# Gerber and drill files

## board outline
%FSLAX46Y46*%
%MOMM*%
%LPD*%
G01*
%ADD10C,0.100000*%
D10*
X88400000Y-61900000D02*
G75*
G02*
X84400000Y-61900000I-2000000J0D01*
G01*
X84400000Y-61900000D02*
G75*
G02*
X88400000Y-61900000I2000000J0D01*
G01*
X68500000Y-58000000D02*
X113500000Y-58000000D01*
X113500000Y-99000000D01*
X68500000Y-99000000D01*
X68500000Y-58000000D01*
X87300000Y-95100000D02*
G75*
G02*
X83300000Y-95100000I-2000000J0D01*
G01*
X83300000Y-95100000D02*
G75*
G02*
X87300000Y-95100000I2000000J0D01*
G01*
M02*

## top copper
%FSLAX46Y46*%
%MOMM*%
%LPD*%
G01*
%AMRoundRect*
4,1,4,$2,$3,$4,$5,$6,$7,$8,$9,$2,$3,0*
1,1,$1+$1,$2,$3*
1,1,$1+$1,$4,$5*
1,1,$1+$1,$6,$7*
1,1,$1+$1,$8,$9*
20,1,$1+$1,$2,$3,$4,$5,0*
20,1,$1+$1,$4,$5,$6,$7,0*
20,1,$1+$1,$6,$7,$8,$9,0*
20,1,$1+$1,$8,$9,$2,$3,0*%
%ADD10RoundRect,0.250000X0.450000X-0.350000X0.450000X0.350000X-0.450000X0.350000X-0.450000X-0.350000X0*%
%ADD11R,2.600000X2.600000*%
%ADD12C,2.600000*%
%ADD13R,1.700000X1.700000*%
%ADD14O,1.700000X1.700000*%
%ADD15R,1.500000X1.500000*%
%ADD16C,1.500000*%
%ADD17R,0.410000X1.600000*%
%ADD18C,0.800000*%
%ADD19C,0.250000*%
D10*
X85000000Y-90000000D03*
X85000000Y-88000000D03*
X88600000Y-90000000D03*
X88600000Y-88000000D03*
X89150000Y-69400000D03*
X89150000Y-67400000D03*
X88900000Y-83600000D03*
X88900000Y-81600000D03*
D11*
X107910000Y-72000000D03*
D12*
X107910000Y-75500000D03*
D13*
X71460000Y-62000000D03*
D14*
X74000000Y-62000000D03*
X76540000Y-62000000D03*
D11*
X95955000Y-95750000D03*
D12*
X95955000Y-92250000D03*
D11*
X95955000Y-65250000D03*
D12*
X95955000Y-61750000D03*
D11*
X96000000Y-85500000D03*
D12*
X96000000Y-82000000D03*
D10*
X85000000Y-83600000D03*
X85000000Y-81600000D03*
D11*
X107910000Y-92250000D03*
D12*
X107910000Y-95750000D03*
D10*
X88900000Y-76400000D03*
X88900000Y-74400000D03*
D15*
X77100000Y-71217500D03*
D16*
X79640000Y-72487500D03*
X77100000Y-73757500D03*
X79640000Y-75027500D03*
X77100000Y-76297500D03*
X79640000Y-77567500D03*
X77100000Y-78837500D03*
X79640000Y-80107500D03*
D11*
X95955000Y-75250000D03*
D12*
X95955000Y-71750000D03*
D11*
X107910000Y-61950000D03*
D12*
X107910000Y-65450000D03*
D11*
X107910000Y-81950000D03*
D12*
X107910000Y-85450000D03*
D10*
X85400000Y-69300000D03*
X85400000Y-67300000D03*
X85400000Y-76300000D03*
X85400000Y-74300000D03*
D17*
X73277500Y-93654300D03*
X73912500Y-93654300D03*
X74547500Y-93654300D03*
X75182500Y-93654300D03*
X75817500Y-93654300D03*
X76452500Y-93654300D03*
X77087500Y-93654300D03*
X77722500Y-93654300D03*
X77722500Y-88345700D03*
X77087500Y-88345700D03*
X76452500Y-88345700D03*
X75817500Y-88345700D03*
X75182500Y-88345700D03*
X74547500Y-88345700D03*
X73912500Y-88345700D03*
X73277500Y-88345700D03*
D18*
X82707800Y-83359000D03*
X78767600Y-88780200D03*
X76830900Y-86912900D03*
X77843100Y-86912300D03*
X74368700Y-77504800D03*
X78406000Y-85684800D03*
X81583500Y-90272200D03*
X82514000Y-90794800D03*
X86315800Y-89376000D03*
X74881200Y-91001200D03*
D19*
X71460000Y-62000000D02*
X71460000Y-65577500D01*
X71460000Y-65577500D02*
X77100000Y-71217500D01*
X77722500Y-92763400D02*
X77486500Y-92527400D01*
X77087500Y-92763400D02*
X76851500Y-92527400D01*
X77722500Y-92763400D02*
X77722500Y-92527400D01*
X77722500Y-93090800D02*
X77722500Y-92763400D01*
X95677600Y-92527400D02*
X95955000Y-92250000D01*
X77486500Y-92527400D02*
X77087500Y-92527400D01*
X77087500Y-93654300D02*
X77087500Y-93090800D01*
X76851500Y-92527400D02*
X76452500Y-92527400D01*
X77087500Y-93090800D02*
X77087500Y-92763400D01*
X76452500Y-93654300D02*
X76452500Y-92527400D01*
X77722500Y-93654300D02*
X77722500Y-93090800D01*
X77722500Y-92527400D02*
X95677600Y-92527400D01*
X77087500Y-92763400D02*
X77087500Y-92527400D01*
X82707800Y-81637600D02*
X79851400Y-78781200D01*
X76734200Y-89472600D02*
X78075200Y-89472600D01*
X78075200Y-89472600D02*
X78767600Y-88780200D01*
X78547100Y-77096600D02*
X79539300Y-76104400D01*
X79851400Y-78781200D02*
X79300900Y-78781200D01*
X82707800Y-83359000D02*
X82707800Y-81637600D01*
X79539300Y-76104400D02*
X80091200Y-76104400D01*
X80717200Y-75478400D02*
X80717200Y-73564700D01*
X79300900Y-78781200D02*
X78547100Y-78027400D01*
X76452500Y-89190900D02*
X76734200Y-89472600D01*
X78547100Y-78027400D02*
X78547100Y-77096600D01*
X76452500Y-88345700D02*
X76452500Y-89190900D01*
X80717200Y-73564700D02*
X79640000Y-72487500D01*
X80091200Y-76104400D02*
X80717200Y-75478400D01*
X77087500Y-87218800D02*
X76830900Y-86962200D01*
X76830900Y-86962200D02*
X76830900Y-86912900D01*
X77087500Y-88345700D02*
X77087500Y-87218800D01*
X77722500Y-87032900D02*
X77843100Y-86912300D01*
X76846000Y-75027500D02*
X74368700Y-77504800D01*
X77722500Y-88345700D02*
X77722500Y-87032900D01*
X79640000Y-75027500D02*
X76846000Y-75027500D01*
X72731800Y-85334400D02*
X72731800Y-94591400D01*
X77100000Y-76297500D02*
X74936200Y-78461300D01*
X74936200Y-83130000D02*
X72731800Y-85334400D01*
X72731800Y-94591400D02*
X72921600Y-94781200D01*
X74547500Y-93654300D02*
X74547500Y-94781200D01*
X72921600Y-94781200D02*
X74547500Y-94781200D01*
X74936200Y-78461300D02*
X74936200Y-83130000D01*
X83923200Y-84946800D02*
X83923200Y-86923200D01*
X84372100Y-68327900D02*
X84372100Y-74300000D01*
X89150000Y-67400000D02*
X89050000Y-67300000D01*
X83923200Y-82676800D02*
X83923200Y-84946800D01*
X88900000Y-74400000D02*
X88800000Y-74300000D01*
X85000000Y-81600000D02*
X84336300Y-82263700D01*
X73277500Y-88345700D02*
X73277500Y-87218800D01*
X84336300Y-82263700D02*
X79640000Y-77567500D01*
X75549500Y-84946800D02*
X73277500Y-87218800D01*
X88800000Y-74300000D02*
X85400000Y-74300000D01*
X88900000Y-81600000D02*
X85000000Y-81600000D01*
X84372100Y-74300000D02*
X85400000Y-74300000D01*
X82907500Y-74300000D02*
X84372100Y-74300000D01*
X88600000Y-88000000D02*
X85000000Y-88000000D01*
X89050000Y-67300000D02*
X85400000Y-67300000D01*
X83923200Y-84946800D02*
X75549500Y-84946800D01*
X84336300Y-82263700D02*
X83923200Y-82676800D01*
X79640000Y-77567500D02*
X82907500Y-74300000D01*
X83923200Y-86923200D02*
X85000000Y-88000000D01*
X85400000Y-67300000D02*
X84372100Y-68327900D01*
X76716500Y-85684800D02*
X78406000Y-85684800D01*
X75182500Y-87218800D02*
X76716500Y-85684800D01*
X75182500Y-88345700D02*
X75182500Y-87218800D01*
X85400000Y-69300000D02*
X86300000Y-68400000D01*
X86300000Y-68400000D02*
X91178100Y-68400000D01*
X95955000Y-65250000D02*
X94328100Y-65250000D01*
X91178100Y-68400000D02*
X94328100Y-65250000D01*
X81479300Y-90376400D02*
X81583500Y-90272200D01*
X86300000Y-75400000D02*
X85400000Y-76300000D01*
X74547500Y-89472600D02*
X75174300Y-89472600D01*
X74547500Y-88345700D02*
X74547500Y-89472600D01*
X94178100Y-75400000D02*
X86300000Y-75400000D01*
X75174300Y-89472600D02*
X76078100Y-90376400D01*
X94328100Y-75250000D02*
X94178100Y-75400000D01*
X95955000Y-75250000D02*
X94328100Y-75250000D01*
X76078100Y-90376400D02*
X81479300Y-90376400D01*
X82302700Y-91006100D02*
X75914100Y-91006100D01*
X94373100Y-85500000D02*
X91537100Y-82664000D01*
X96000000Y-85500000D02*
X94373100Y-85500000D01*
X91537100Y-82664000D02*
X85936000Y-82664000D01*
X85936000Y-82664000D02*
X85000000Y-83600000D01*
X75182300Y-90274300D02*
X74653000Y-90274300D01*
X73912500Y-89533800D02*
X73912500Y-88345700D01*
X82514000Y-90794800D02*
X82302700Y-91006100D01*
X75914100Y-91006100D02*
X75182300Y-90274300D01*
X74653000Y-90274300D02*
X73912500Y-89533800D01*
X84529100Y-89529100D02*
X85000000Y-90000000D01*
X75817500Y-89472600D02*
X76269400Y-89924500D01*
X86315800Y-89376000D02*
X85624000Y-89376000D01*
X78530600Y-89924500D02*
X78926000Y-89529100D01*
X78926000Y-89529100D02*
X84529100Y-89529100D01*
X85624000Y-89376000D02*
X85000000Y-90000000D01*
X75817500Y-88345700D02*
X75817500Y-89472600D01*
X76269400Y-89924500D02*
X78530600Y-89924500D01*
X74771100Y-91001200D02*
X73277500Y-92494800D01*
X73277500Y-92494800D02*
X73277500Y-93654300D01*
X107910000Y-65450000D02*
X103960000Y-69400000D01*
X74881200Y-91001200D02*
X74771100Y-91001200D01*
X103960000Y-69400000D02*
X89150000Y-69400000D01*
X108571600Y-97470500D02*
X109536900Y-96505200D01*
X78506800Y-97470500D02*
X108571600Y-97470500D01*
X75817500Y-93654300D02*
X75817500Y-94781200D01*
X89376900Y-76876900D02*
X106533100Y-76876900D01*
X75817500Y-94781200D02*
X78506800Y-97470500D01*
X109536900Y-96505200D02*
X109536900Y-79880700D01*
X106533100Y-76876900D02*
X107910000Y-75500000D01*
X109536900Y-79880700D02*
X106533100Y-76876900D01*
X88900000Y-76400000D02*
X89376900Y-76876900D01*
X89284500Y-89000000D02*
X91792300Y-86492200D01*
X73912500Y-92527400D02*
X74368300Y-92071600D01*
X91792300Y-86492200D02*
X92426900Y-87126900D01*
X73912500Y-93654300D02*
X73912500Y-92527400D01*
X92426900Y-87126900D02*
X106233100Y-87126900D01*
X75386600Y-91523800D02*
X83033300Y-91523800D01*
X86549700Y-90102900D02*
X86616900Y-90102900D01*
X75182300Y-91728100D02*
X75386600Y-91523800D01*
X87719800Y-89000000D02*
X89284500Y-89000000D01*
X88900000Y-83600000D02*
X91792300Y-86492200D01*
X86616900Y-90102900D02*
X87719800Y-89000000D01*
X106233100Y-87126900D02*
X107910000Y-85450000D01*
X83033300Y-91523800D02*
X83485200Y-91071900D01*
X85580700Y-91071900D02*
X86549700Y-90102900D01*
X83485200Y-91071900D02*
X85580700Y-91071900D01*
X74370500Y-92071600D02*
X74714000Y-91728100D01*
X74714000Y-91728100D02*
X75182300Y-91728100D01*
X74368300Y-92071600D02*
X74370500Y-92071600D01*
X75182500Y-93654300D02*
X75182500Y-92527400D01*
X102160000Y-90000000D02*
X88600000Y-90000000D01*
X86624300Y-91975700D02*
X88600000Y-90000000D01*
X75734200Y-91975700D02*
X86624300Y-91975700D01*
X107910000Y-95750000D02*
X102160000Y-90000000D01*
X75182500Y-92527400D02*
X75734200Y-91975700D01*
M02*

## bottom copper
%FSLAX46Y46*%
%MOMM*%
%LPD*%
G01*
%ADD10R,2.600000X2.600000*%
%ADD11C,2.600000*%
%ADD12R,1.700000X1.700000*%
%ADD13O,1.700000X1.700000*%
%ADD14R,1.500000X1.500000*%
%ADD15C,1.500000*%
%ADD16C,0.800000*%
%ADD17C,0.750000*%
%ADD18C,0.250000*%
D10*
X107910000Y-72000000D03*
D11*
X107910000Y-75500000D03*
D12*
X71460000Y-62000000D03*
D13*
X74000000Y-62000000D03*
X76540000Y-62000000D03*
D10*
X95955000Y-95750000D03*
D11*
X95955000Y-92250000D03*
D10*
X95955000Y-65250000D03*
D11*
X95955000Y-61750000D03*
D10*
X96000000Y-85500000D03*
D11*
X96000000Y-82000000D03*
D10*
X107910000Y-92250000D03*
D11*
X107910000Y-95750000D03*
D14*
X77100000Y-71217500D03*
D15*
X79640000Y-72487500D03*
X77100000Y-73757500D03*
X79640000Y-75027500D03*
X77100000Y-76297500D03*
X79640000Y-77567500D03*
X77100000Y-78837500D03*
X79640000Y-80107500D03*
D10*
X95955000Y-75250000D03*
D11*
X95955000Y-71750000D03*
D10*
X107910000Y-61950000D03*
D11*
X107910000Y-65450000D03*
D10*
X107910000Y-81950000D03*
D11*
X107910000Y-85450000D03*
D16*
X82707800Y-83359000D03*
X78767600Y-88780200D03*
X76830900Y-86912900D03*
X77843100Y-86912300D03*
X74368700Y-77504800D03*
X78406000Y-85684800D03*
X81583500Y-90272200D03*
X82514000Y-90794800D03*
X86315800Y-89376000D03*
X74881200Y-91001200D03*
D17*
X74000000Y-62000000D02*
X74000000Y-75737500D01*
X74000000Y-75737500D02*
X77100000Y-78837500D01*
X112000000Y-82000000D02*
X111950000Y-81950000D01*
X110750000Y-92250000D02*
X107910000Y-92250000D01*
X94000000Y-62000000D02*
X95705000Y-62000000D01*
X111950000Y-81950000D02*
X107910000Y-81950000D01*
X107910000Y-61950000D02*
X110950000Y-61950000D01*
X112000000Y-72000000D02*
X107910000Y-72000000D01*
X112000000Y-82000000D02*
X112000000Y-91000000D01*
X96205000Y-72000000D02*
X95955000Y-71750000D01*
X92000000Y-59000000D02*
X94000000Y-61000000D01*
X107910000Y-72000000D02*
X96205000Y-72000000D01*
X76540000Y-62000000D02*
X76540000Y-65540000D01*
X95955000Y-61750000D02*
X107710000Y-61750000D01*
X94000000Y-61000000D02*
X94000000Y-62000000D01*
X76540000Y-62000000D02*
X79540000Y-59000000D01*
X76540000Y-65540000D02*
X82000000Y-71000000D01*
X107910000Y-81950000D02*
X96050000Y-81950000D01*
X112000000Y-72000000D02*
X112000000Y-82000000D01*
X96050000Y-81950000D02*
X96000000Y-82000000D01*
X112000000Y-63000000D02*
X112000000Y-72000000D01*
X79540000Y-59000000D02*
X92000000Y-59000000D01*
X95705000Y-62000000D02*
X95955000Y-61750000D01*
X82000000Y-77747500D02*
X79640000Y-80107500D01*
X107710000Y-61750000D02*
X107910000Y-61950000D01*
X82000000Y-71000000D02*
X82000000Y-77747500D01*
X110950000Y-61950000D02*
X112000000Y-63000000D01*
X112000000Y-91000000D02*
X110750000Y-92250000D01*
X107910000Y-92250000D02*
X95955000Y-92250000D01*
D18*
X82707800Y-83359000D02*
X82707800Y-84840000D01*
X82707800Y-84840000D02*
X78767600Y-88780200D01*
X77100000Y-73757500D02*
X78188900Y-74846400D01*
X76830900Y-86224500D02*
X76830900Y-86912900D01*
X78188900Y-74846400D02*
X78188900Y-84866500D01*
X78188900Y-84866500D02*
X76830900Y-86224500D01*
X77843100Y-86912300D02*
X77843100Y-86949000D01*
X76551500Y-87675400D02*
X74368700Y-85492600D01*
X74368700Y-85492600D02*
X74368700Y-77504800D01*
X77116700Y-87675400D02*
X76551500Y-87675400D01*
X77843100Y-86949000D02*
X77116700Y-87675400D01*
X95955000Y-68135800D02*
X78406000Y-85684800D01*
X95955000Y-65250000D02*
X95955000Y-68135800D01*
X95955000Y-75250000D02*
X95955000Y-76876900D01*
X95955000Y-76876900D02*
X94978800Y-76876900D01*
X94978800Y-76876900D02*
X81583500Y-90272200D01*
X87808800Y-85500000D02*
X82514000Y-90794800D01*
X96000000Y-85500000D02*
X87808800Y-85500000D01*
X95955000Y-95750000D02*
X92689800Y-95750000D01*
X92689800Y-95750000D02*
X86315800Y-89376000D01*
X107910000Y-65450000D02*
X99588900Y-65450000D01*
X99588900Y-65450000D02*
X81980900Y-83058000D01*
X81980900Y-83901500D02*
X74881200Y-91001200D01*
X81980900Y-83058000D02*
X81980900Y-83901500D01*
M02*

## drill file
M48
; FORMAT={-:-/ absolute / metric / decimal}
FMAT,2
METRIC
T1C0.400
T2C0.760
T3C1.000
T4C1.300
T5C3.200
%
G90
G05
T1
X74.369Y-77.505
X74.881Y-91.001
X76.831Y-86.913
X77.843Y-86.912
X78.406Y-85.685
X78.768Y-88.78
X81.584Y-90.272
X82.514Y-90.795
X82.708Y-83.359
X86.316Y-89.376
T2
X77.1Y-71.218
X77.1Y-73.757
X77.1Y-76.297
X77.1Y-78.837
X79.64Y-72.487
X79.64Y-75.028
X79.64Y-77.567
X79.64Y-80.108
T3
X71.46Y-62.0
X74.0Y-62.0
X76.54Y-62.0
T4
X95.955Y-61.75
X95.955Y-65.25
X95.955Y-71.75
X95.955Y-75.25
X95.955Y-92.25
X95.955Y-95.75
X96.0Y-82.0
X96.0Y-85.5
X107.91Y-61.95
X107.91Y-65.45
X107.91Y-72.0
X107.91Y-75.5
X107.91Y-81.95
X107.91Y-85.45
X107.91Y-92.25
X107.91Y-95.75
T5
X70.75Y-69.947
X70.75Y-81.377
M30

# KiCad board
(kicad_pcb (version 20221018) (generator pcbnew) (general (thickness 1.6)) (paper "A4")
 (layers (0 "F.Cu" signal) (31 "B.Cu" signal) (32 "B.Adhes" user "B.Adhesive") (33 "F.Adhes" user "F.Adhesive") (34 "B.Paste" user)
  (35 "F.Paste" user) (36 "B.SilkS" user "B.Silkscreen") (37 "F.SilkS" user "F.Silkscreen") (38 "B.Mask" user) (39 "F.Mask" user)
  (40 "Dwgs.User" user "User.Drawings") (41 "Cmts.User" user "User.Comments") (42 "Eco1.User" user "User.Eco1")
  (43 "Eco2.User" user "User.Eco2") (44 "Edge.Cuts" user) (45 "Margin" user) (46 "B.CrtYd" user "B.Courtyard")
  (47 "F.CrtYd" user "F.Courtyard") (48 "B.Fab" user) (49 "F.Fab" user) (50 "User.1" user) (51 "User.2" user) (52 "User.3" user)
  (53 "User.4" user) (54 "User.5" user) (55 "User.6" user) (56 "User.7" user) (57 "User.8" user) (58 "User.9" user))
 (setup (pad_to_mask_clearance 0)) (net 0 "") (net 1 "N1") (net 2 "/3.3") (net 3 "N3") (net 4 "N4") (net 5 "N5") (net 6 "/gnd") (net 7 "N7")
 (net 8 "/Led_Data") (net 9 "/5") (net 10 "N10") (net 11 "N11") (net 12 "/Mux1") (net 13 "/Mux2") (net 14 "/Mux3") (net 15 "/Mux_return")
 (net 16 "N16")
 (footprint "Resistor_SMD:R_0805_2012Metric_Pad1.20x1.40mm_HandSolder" (layer "F.Cu") (at 85 89 90)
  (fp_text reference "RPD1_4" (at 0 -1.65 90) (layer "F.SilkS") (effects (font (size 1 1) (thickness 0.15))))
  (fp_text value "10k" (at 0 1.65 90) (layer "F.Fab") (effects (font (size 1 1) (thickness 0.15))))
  (pad "1" smd roundrect (at -1 0 90) (size 1.2 1.4) (layers "F.Cu" "F.Paste" "F.Mask") (roundrect_rratio 0.2083333333) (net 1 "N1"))
  (pad "2" smd roundrect (at 1 0 90) (size 1.2 1.4) (layers "F.Cu" "F.Paste" "F.Mask") (roundrect_rratio 0.2083333333) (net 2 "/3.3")))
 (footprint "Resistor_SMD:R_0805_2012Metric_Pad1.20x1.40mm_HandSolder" (layer "F.Cu") (at 88.6 89 90)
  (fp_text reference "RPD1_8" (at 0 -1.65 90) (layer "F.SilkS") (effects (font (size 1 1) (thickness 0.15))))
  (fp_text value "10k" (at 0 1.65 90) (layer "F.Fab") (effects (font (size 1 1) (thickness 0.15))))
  (pad "1" smd roundrect (at -1 0 90) (size 1.2 1.4) (layers "F.Cu" "F.Paste" "F.Mask") (roundrect_rratio 0.2083333333) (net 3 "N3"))
  (pad "2" smd roundrect (at 1 0 90) (size 1.2 1.4) (layers "F.Cu" "F.Paste" "F.Mask") (roundrect_rratio 0.2083333333) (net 2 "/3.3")))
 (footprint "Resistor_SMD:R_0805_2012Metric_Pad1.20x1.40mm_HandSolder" (layer "F.Cu") (at 89.15 68.4 90)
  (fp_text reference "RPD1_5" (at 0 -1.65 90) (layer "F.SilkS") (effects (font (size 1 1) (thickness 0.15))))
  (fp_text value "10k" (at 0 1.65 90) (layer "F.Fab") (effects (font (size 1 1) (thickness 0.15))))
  (pad "1" smd roundrect (at -1 0 90) (size 1.2 1.4) (layers "F.Cu" "F.Paste" "F.Mask") (roundrect_rratio 0.2083333333) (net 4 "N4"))
  (pad "2" smd roundrect (at 1 0 90) (size 1.2 1.4) (layers "F.Cu" "F.Paste" "F.Mask") (roundrect_rratio 0.2083333333) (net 2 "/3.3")))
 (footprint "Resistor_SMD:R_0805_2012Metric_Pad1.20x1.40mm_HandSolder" (layer "F.Cu") (at 88.9 82.6 90)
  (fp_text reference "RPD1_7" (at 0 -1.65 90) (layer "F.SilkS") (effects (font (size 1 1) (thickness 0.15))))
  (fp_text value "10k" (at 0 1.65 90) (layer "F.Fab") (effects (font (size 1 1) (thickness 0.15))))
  (pad "1" smd roundrect (at -1 0 90) (size 1.2 1.4) (layers "F.Cu" "F.Paste" "F.Mask") (roundrect_rratio 0.2083333333) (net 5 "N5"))
  (pad "2" smd roundrect (at 1 0 90) (size 1.2 1.4) (layers "F.Cu" "F.Paste" "F.Mask") (roundrect_rratio 0.2083333333) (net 2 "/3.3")))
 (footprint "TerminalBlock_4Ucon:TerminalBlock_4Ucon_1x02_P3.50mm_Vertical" (layer "F.Cu") (at 107.91 72 -90)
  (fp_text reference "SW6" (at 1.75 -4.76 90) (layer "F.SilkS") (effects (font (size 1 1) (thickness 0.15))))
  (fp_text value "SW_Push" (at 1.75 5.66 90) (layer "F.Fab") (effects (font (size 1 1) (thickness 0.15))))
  (pad "1" thru_hole rect (at 0 0 270) (size 2.6 2.6) (drill 1.3) (layers "*.Cu" "*.Mask") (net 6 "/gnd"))
  (pad "2" thru_hole circle (at 3.5 0 270) (size 2.6 2.6) (drill 1.3) (layers "*.Cu" "*.Mask") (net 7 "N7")))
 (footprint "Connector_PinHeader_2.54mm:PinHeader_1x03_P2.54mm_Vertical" (layer "F.Cu") (at 71.46 62 90)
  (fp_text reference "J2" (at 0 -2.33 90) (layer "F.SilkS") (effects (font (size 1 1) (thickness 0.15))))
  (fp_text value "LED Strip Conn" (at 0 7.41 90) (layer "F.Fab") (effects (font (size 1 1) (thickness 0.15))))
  (pad "1" thru_hole rect (at 0 0 90) (size 1.7 1.7) (drill 1) (layers "*.Cu" "*.Mask") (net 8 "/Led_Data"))
  (pad "2" thru_hole oval (at 0 2.54 90) (size 1.7 1.7) (drill 1) (layers "*.Cu" "*.Mask") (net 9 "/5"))
  (pad "3" thru_hole oval (at 0 5.08 90) (size 1.7 1.7) (drill 1) (layers "*.Cu" "*.Mask") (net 6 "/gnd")))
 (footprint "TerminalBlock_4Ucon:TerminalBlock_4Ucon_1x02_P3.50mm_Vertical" (layer "F.Cu") (at 95.955 95.75 90)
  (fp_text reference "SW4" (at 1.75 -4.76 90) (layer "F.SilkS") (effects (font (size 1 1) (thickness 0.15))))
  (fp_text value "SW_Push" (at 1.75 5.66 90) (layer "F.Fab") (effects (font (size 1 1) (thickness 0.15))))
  (pad "1" thru_hole rect (at 0 0 90) (size 2.6 2.6) (drill 1.3) (layers "*.Cu" "*.Mask") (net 1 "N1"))
  (pad "2" thru_hole circle (at 3.5 0 90) (size 2.6 2.6) (drill 1.3) (layers "*.Cu" "*.Mask") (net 6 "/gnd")))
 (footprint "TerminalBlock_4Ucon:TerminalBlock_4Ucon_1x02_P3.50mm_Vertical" (layer "F.Cu") (at 95.955 65.25 90)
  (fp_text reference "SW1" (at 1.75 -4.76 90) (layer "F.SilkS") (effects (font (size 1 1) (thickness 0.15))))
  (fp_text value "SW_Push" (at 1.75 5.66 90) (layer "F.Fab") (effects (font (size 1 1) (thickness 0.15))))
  (pad "1" thru_hole rect (at 0 0 90) (size 2.6 2.6) (drill 1.3) (layers "*.Cu" "*.Mask") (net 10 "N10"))
  (pad "2" thru_hole circle (at 3.5 0 90) (size 2.6 2.6) (drill 1.3) (layers "*.Cu" "*.Mask") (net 6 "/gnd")))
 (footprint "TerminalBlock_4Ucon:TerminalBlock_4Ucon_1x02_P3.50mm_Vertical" (layer "F.Cu") (at 96 85.5 90)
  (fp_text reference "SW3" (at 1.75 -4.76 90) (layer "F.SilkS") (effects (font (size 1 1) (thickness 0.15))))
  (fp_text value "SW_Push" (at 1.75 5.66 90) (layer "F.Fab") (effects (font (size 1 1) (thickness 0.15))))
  (pad "1" thru_hole rect (at 0 0 90) (size 2.6 2.6) (drill 1.3) (layers "*.Cu" "*.Mask") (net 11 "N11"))
  (pad "2" thru_hole circle (at 3.5 0 90) (size 2.6 2.6) (drill 1.3) (layers "*.Cu" "*.Mask") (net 6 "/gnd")))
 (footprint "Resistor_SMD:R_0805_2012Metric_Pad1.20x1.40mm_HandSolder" (layer "F.Cu") (at 85 82.6 90)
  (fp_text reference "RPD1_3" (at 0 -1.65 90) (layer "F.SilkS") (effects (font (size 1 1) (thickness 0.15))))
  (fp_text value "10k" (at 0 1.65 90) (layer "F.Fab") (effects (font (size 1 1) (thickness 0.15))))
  (pad "1" smd roundrect (at -1 0 90) (size 1.2 1.4) (layers "F.Cu" "F.Paste" "F.Mask") (roundrect_rratio 0.2083333333) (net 11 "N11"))
  (pad "2" smd roundrect (at 1 0 90) (size 1.2 1.4) (layers "F.Cu" "F.Paste" "F.Mask") (roundrect_rratio 0.2083333333) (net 2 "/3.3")))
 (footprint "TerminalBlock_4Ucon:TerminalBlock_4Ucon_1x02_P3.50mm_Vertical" (layer "F.Cu") (at 107.91 92.25 -90)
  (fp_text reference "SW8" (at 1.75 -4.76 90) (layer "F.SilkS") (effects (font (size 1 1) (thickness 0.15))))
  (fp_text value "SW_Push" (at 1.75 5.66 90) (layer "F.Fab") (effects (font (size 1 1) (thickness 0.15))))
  (pad "1" thru_hole rect (at 0 0 270) (size 2.6 2.6) (drill 1.3) (layers "*.Cu" "*.Mask") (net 6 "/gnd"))
  (pad "2" thru_hole circle (at 3.5 0 270) (size 2.6 2.6) (drill 1.3) (layers "*.Cu" "*.Mask") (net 3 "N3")))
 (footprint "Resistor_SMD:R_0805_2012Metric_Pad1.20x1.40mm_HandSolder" (layer "F.Cu") (at 88.9 75.4 90)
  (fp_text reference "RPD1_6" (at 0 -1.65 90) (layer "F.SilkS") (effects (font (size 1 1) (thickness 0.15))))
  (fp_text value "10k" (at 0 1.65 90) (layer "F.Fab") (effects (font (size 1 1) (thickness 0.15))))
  (pad "1" smd roundrect (at -1 0 90) (size 1.2 1.4) (layers "F.Cu" "F.Paste" "F.Mask") (roundrect_rratio 0.2083333333) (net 7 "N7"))
  (pad "2" smd roundrect (at 1 0 90) (size 1.2 1.4) (layers "F.Cu" "F.Paste" "F.Mask") (roundrect_rratio 0.2083333333) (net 2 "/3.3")))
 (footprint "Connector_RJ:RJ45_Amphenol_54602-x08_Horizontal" (layer "F.Cu") (at 77.1 71.2175 -90)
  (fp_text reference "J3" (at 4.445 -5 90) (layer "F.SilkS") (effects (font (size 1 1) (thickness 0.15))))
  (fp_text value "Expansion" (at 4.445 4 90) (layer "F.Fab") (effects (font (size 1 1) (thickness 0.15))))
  (pad "" np_thru_hole circle (at -1.27 6.35 270) (size 3.2 3.2) (drill 3.2) (layers "*.Cu" "*.Mask"))
  (pad "" np_thru_hole circle (at 10.16 6.35 270) (size 3.2 3.2) (drill 3.2) (layers "*.Cu" "*.Mask"))
  (pad "1" thru_hole rect (at 0 0 270) (size 1.5 1.5) (drill 0.76) (layers "*.Cu" "*.Mask") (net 8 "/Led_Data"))
  (pad "2" thru_hole circle (at 1.27 -2.54 270) (size 1.5 1.5) (drill 0.76) (layers "*.Cu" "*.Mask") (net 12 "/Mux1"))
  (pad "3" thru_hole circle (at 2.54 0 270) (size 1.5 1.5) (drill 0.76) (layers "*.Cu" "*.Mask") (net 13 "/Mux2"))
  (pad "4" thru_hole circle (at 3.81 -2.54 270) (size 1.5 1.5) (drill 0.76) (layers "*.Cu" "*.Mask") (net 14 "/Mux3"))
  (pad "5" thru_hole circle (at 5.08 0 270) (size 1.5 1.5) (drill 0.76) (layers "*.Cu" "*.Mask") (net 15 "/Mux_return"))
  (pad "6" thru_hole circle (at 6.35 -2.54 270) (size 1.5 1.5) (drill 0.76) (layers "*.Cu" "*.Mask") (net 2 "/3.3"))
  (pad "7" thru_hole circle (at 7.62 0 270) (size 1.5 1.5) (drill 0.76) (layers "*.Cu" "*.Mask") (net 9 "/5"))
  (pad "8" thru_hole circle (at 8.89 -2.54 270) (size 1.5 1.5) (drill 0.76) (layers "*.Cu" "*.Mask") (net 6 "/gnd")))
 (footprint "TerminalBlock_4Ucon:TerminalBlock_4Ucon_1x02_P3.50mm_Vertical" (layer "F.Cu") (at 95.955 75.25 90)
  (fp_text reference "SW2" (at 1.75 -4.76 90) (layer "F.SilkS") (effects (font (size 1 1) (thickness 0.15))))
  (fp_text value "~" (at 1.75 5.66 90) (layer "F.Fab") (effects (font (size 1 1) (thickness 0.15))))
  (pad "1" thru_hole rect (at 0 0 90) (size 2.6 2.6) (drill 1.3) (layers "*.Cu" "*.Mask") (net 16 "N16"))
  (pad "2" thru_hole circle (at 3.5 0 90) (size 2.6 2.6) (drill 1.3) (layers "*.Cu" "*.Mask") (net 6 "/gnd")))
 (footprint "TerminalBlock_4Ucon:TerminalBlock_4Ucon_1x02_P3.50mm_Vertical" (layer "F.Cu") (at 107.91 61.95 -90)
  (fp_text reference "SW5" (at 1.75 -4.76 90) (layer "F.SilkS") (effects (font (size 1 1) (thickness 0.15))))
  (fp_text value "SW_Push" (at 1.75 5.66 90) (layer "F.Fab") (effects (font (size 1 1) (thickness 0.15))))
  (pad "1" thru_hole rect (at 0 0 270) (size 2.6 2.6) (drill 1.3) (layers "*.Cu" "*.Mask") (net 6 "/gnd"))
  (pad "2" thru_hole circle (at 3.5 0 270) (size 2.6 2.6) (drill 1.3) (layers "*.Cu" "*.Mask") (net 4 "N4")))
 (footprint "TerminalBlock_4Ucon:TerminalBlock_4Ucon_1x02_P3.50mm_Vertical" (layer "F.Cu") (at 107.91 81.95 -90)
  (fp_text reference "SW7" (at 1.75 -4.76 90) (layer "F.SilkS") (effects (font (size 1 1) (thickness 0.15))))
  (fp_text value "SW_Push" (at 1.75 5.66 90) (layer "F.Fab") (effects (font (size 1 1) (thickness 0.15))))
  (pad "1" thru_hole rect (at 0 0 270) (size 2.6 2.6) (drill 1.3) (layers "*.Cu" "*.Mask") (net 6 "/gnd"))
  (pad "2" thru_hole circle (at 3.5 0 270) (size 2.6 2.6) (drill 1.3) (layers "*.Cu" "*.Mask") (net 5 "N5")))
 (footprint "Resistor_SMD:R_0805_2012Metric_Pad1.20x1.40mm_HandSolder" (layer "F.Cu") (at 85.4 68.3 90)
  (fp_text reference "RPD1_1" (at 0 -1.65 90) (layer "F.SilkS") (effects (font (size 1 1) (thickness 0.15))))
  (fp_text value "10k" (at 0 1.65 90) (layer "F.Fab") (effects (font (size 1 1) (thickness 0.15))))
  (pad "1" smd roundrect (at -1 0 90) (size 1.2 1.4) (layers "F.Cu" "F.Paste" "F.Mask") (roundrect_rratio 0.2083333333) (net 10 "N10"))
  (pad "2" smd roundrect (at 1 0 90) (size 1.2 1.4) (layers "F.Cu" "F.Paste" "F.Mask") (roundrect_rratio 0.2083333333) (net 2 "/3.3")))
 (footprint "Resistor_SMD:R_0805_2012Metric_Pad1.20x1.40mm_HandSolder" (layer "F.Cu") (at 85.4 75.3 90)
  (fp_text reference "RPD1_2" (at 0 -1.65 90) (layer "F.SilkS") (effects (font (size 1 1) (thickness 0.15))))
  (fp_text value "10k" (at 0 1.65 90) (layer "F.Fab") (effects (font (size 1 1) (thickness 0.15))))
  (pad "1" smd roundrect (at -1 0 90) (size 1.2 1.4) (layers "F.Cu" "F.Paste" "F.Mask") (roundrect_rratio 0.2083333333) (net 16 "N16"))
  (pad "2" smd roundrect (at 1 0 90) (size 1.2 1.4) (layers "F.Cu" "F.Paste" "F.Mask") (roundrect_rratio 0.2083333333) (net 2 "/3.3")))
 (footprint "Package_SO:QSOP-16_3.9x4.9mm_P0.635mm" (layer "F.Cu") (at 75.5 91 90)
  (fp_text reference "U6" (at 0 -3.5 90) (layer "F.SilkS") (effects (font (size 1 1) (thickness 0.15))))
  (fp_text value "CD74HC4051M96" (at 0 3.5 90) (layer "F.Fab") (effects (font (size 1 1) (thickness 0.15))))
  (pad "1" smd rect (at -2.6543 -2.2225 90) (size 1.6 0.41) (layers "F.Cu" "F.Paste" "F.Mask") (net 4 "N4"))
  (pad "2" smd rect (at -2.6543 -1.5875 90) (size 1.6 0.41) (layers "F.Cu" "F.Paste" "F.Mask") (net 5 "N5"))
  (pad "3" smd rect (at -2.6543 -0.9525 90) (size 1.6 0.41) (layers "F.Cu" "F.Paste" "F.Mask") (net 15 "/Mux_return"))
  (pad "4" smd rect (at -2.6543 -0.3175 90) (size 1.6 0.41) (layers "F.Cu" "F.Paste" "F.Mask") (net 3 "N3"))
  (pad "5" smd rect (at -2.6543 0.3175 90) (size 1.6 0.41) (layers "F.Cu" "F.Paste" "F.Mask") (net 7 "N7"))
  (pad "6" smd rect (at -2.6543 0.9525 90) (size 1.6 0.41) (layers "F.Cu" "F.Paste" "F.Mask") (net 6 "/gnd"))
  (pad "7" smd rect (at -2.6543 1.5875 90) (size 1.6 0.41) (layers "F.Cu" "F.Paste" "F.Mask") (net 6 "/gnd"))
  (pad "8" smd rect (at -2.6543 2.2225 90) (size 1.6 0.41) (layers "F.Cu" "F.Paste" "F.Mask") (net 6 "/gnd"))
  (pad "9" smd rect (at 2.6543 2.2225 90) (size 1.6 0.41) (layers "F.Cu" "F.Paste" "F.Mask") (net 14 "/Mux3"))
  (pad "10" smd rect (at 2.6543 1.5875 90) (size 1.6 0.41) (layers "F.Cu" "F.Paste" "F.Mask") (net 13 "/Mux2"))
  (pad "11" smd rect (at 2.6543 0.9525 90) (size 1.6 0.41) (layers "F.Cu" "F.Paste" "F.Mask") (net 12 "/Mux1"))
  (pad "12" smd rect (at 2.6543 0.3175 90) (size 1.6 0.41) (layers "F.Cu" "F.Paste" "F.Mask") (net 1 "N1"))
  (pad "13" smd rect (at 2.6543 -0.3175 90) (size 1.6 0.41) (layers "F.Cu" "F.Paste" "F.Mask") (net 10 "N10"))
  (pad "14" smd rect (at 2.6543 -0.9525 90) (size 1.6 0.41) (layers "F.Cu" "F.Paste" "F.Mask") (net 16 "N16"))
  (pad "15" smd rect (at 2.6543 -1.5875 90) (size 1.6 0.41) (layers "F.Cu" "F.Paste" "F.Mask") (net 11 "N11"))
  (pad "16" smd rect (at 2.6543 -2.2225 90) (size 1.6 0.41) (layers "F.Cu" "F.Paste" "F.Mask") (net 2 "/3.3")))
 (gr_circle (center 86.4 61.9) (end 88.4 61.9) (stroke (width 0.1) (type default)) (fill none) (layer "Edge.Cuts"))
 (gr_rect (start 68.5 58) (end 113.5 99) (stroke (width 0.1) (type default)) (fill none) (layer "Edge.Cuts"))
 (gr_circle (center 85.3 95.1) (end 87.3 95.1) (stroke (width 0.1) (type default)) (fill none) (layer "Edge.Cuts"))
 (segment (start 71.46 62) (end 71.46 65.5775) (width 0.25) (layer "F.Cu") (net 8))
 (segment (start 71.46 65.5775) (end 77.1 71.2175) (width 0.25) (layer "F.Cu") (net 8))
 (segment (start 74 62) (end 74 75.7375) (width 0.75) (layer "B.Cu") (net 9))
 (segment (start 74 75.7375) (end 77.1 78.8375) (width 0.75) (layer "B.Cu") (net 9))
 (segment (start 77.7225 92.7634) (end 77.4865 92.5274) (width 0.25) (layer "F.Cu") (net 6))
 (segment (start 77.0875 92.7634) (end 76.8515 92.5274) (width 0.25) (layer "F.Cu") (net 6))
 (segment (start 77.7225 92.7634) (end 77.7225 92.5274) (width 0.25) (layer "F.Cu") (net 6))
 (segment (start 77.7225 93.0908) (end 77.7225 92.7634) (width 0.25) (layer "F.Cu") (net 6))
 (segment (start 95.6776 92.5274) (end 95.955 92.25) (width 0.25) (layer "F.Cu") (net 6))
 (segment (start 77.4865 92.5274) (end 77.0875 92.5274) (width 0.25) (layer "F.Cu") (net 6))
 (segment (start 77.0875 93.6543) (end 77.0875 93.0908) (width 0.25) (layer "F.Cu") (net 6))
 (segment (start 76.8515 92.5274) (end 76.4525 92.5274) (width 0.25) (layer "F.Cu") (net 6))
 (segment (start 77.0875 93.0908) (end 77.0875 92.7634) (width 0.25) (layer "F.Cu") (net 6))
 (segment (start 76.4525 93.6543) (end 76.4525 92.5274) (width 0.25) (layer "F.Cu") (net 6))
 (segment (start 77.7225 93.6543) (end 77.7225 93.0908) (width 0.25) (layer "F.Cu") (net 6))
 (segment (start 77.7225 92.5274) (end 95.6776 92.5274) (width 0.25) (layer "F.Cu") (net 6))
 (segment (start 77.0875 92.7634) (end 77.0875 92.5274) (width 0.25) (layer "F.Cu") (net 6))
 (segment (start 112 82) (end 111.95 81.95) (width 0.75) (layer "B.Cu") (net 6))
 (segment (start 110.75 92.25) (end 107.91 92.25) (width 0.75) (layer "B.Cu") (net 6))
 (segment (start 94 62) (end 95.705 62) (width 0.75) (layer "B.Cu") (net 6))
 (segment (start 111.95 81.95) (end 107.91 81.95) (width 0.75) (layer "B.Cu") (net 6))
 (segment (start 107.91 61.95) (end 110.95 61.95) (width 0.75) (layer "B.Cu") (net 6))
 (segment (start 112 72) (end 107.91 72) (width 0.75) (layer "B.Cu") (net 6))
 (segment (start 112 82) (end 112 91) (width 0.75) (layer "B.Cu") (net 6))
 (segment (start 96.205 72) (end 95.955 71.75) (width 0.75) (layer "B.Cu") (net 6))
 (segment (start 92 59) (end 94 61) (width 0.75) (layer "B.Cu") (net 6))
 (segment (start 107.91 72) (end 96.205 72) (width 0.75) (layer "B.Cu") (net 6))
 (segment (start 76.54 62) (end 76.54 65.54) (width 0.75) (layer "B.Cu") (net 6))
 (segment (start 95.955 61.75) (end 107.71 61.75) (width 0.75) (layer "B.Cu") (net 6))
 (segment (start 94 61) (end 94 62) (width 0.75) (layer "B.Cu") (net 6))
 (segment (start 76.54 62) (end 79.54 59) (width 0.75) (layer "B.Cu") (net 6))
 (segment (start 76.54 65.54) (end 82 71) (width 0.75) (layer "B.Cu") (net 6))
 (segment (start 107.91 81.95) (end 96.05 81.95) (width 0.75) (layer "B.Cu") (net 6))
 (segment (start 112 72) (end 112 82) (width 0.75) (layer "B.Cu") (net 6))
 (segment (start 96.05 81.95) (end 96 82) (width 0.75) (layer "B.Cu") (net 6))
 (segment (start 112 63) (end 112 72) (width 0.75) (layer "B.Cu") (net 6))
 (segment (start 79.54 59) (end 92 59) (width 0.75) (layer "B.Cu") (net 6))
 (segment (start 95.705 62) (end 95.955 61.75) (width 0.75) (layer "B.Cu") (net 6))
 (segment (start 82 77.7475) (end 79.64 80.1075) (width 0.75) (layer "B.Cu") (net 6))
 (segment (start 107.71 61.75) (end 107.91 61.95) (width 0.75) (layer "B.Cu") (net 6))
 (segment (start 82 71) (end 82 77.7475) (width 0.75) (layer "B.Cu") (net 6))
 (segment (start 110.95 61.95) (end 112 63) (width 0.75) (layer "B.Cu") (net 6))
 (segment (start 112 91) (end 110.75 92.25) (width 0.75) (layer "B.Cu") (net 6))
 (segment (start 107.91 92.25) (end 95.955 92.25) (width 0.75) (layer "B.Cu") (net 6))
 (segment (start 82.7078 81.6376) (end 79.8514 78.7812) (width 0.25) (layer "F.Cu") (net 12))
 (segment (start 76.7342 89.4726) (end 78.0752 89.4726) (width 0.25) (layer "F.Cu") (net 12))
 (segment (start 78.0752 89.4726) (end 78.7676 88.7802) (width 0.25) (layer "F.Cu") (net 12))
 (segment (start 78.5471 77.0966) (end 79.5393 76.1044) (width 0.25) (layer "F.Cu") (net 12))
 (segment (start 79.8514 78.7812) (end 79.3009 78.7812) (width 0.25) (layer "F.Cu") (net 12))
 (segment (start 82.7078 83.359) (end 82.7078 81.6376) (width 0.25) (layer "F.Cu") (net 12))
 (segment (start 79.5393 76.1044) (end 80.0912 76.1044) (width 0.25) (layer "F.Cu") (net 12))
 (segment (start 80.7172 75.4784) (end 80.7172 73.5647) (width 0.25) (layer "F.Cu") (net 12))
 (segment (start 79.3009 78.7812) (end 78.5471 78.0274) (width 0.25) (layer "F.Cu") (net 12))
 (segment (start 76.4525 89.1909) (end 76.7342 89.4726) (width 0.25) (layer "F.Cu") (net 12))
 (segment (start 78.5471 78.0274) (end 78.5471 77.0966) (width 0.25) (layer "F.Cu") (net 12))
 (segment (start 76.4525 88.3457) (end 76.4525 89.1909) (width 0.25) (layer "F.Cu") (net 12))
 (segment (start 80.7172 73.5647) (end 79.64 72.4875) (width 0.25) (layer "F.Cu") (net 12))
 (segment (start 80.0912 76.1044) (end 80.7172 75.4784) (width 0.25) (layer "F.Cu") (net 12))
 (via (at 82.7078 83.359) (size 0.8) (drill 0.4) (layers "F.Cu" "B.Cu") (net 12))
 (via (at 78.7676 88.7802) (size 0.8) (drill 0.4) (layers "F.Cu" "B.Cu") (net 12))
 (segment (start 82.7078 83.359) (end 82.7078 84.84) (width 0.25) (layer "B.Cu") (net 12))
 (segment (start 82.7078 84.84) (end 78.7676 88.7802) (width 0.25) (layer "B.Cu") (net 12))
 (segment (start 77.0875 87.2188) (end 76.8309 86.9622) (width 0.25) (layer "F.Cu") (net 13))
 (segment (start 76.8309 86.9622) (end 76.8309 86.9129) (width 0.25) (layer "F.Cu") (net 13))
 (segment (start 77.0875 88.3457) (end 77.0875 87.2188) (width 0.25) (layer "F.Cu") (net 13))
 (via (at 76.8309 86.9129) (size 0.8) (drill 0.4) (layers "F.Cu" "B.Cu") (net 13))
 (segment (start 77.1 73.7575) (end 78.1889 74.8464) (width 0.25) (layer "B.Cu") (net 13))
 (segment (start 76.8309 86.2245) (end 76.8309 86.9129) (width 0.25) (layer "B.Cu") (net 13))
 (segment (start 78.1889 74.8464) (end 78.1889 84.8665) (width 0.25) (layer "B.Cu") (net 13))
 (segment (start 78.1889 84.8665) (end 76.8309 86.2245) (width 0.25) (layer "B.Cu") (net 13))
 (segment (start 77.7225 87.0329) (end 77.8431 86.9123) (width 0.25) (layer "F.Cu") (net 14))
 (segment (start 76.846 75.0275) (end 74.3687 77.5048) (width 0.25) (layer "F.Cu") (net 14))
 (segment (start 77.7225 88.3457) (end 77.7225 87.0329) (width 0.25) (layer "F.Cu") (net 14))
 (segment (start 79.64 75.0275) (end 76.846 75.0275) (width 0.25) (layer "F.Cu") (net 14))
 (via (at 77.8431 86.9123) (size 0.8) (drill 0.4) (layers "F.Cu" "B.Cu") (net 14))
 (via (at 74.3687 77.5048) (size 0.8) (drill 0.4) (layers "F.Cu" "B.Cu") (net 14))
 (segment (start 77.8431 86.9123) (end 77.8431 86.949) (width 0.25) (layer "B.Cu") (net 14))
 (segment (start 76.5515 87.6754) (end 74.3687 85.4926) (width 0.25) (layer "B.Cu") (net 14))
 (segment (start 74.3687 85.4926) (end 74.3687 77.5048) (width 0.25) (layer "B.Cu") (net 14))
 (segment (start 77.1167 87.6754) (end 76.5515 87.6754) (width 0.25) (layer "B.Cu") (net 14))
 (segment (start 77.8431 86.949) (end 77.1167 87.6754) (width 0.25) (layer "B.Cu") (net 14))
 (segment (start 72.7318 85.3344) (end 72.7318 94.5914) (width 0.25) (layer "F.Cu") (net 15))
 (segment (start 77.1 76.2975) (end 74.9362 78.4613) (width 0.25) (layer "F.Cu") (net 15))
 (segment (start 74.9362 83.13) (end 72.7318 85.3344) (width 0.25) (layer "F.Cu") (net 15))
 (segment (start 72.7318 94.5914) (end 72.9216 94.7812) (width 0.25) (layer "F.Cu") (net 15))
 (segment (start 74.5475 93.6543) (end 74.5475 94.7812) (width 0.25) (layer "F.Cu") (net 15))
 (segment (start 72.9216 94.7812) (end 74.5475 94.7812) (width 0.25) (layer "F.Cu") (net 15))
 (segment (start 74.9362 78.4613) (end 74.9362 83.13) (width 0.25) (layer "F.Cu") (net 15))
 (segment (start 83.9232 84.9468) (end 83.9232 86.9232) (width 0.25) (layer "F.Cu") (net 2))
 (segment (start 84.3721 68.3279) (end 84.3721 74.3) (width 0.25) (layer "F.Cu") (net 2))
 (segment (start 89.15 67.4) (end 89.05 67.3) (width 0.25) (layer "F.Cu") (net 2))
 (segment (start 83.9232 82.6768) (end 83.9232 84.9468) (width 0.25) (layer "F.Cu") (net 2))
 (segment (start 88.9 74.4) (end 88.8 74.3) (width 0.25) (layer "F.Cu") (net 2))
 (segment (start 85 81.6) (end 84.3363 82.2637) (width 0.25) (layer "F.Cu") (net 2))
 (segment (start 73.2775 88.3457) (end 73.2775 87.2188) (width 0.25) (layer "F.Cu") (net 2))
 (segment (start 84.3363 82.2637) (end 79.64 77.5675) (width 0.25) (layer "F.Cu") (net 2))
 (segment (start 75.5495 84.9468) (end 73.2775 87.2188) (width 0.25) (layer "F.Cu") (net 2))
 (segment (start 88.8 74.3) (end 85.4 74.3) (width 0.25) (layer "F.Cu") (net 2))
 (segment (start 88.9 81.6) (end 85 81.6) (width 0.25) (layer "F.Cu") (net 2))
 (segment (start 84.3721 74.3) (end 85.4 74.3) (width 0.25) (layer "F.Cu") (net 2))
 (segment (start 82.9075 74.3) (end 84.3721 74.3) (width 0.25) (layer "F.Cu") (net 2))
 (segment (start 88.6 88) (end 85 88) (width 0.25) (layer "F.Cu") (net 2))
 (segment (start 89.05 67.3) (end 85.4 67.3) (width 0.25) (layer "F.Cu") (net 2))
 (segment (start 83.9232 84.9468) (end 75.5495 84.9468) (width 0.25) (layer "F.Cu") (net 2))
 (segment (start 84.3363 82.2637) (end 83.9232 82.6768) (width 0.25) (layer "F.Cu") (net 2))
 (segment (start 79.64 77.5675) (end 82.9075 74.3) (width 0.25) (layer "F.Cu") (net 2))
 (segment (start 83.9232 86.9232) (end 85 88) (width 0.25) (layer "F.Cu") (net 2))
 (segment (start 85.4 67.3) (end 84.3721 68.3279) (width 0.25) (layer "F.Cu") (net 2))
 (segment (start 76.7165 85.6848) (end 78.406 85.6848) (width 0.25) (layer "F.Cu") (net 10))
 (segment (start 75.1825 87.2188) (end 76.7165 85.6848) (width 0.25) (layer "F.Cu") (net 10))
 (segment (start 75.1825 88.3457) (end 75.1825 87.2188) (width 0.25) (layer "F.Cu") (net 10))
 (segment (start 85.4 69.3) (end 86.3 68.4) (width 0.25) (layer "F.Cu") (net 10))
 (segment (start 86.3 68.4) (end 91.1781 68.4) (width 0.25) (layer "F.Cu") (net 10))
 (segment (start 95.955 65.25) (end 94.3281 65.25) (width 0.25) (layer "F.Cu") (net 10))
 (segment (start 91.1781 68.4) (end 94.3281 65.25) (width 0.25) (layer "F.Cu") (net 10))
 (via (at 78.406 85.6848) (size 0.8) (drill 0.4) (layers "F.Cu" "B.Cu") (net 10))
 (segment (start 95.955 68.1358) (end 78.406 85.6848) (width 0.25) (layer "B.Cu") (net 10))
 (segment (start 95.955 65.25) (end 95.955 68.1358) (width 0.25) (layer "B.Cu") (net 10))
 (segment (start 81.4793 90.3764) (end 81.5835 90.2722) (width 0.25) (layer "F.Cu") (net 16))
 (segment (start 86.3 75.4) (end 85.4 76.3) (width 0.25) (layer "F.Cu") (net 16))
 (segment (start 74.5475 89.4726) (end 75.1743 89.4726) (width 0.25) (layer "F.Cu") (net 16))
 (segment (start 74.5475 88.3457) (end 74.5475 89.4726) (width 0.25) (layer "F.Cu") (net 16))
 (segment (start 94.1781 75.4) (end 86.3 75.4) (width 0.25) (layer "F.Cu") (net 16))
 (segment (start 75.1743 89.4726) (end 76.0781 90.3764) (width 0.25) (layer "F.Cu") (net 16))
 (segment (start 94.3281 75.25) (end 94.1781 75.4) (width 0.25) (layer "F.Cu") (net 16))
 (segment (start 95.955 75.25) (end 94.3281 75.25) (width 0.25) (layer "F.Cu") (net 16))
 (segment (start 76.0781 90.3764) (end 81.4793 90.3764) (width 0.25) (layer "F.Cu") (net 16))
 (via (at 81.5835 90.2722) (size 0.8) (drill 0.4) (layers "F.Cu" "B.Cu") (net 16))
 (segment (start 95.955 75.25) (end 95.955 76.8769) (width 0.25) (layer "B.Cu") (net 16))
 (segment (start 95.955 76.8769) (end 94.9788 76.8769) (width 0.25) (layer "B.Cu") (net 16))
 (segment (start 94.9788 76.8769) (end 81.5835 90.2722) (width 0.25) (layer "B.Cu") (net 16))
 (segment (start 82.3027 91.0061) (end 75.9141 91.0061) (width 0.25) (layer "F.Cu") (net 11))
 (segment (start 94.3731 85.5) (end 91.5371 82.664) (width 0.25) (layer "F.Cu") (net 11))
 (segment (start 96 85.5) (end 94.3731 85.5) (width 0.25) (layer "F.Cu") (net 11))
 (segment (start 91.5371 82.664) (end 85.936 82.664) (width 0.25) (layer "F.Cu") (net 11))
 (segment (start 85.936 82.664) (end 85 83.6) (width 0.25) (layer "F.Cu") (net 11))
 (segment (start 75.1823 90.2743) (end 74.653 90.2743) (width 0.25) (layer "F.Cu") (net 11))
 (segment (start 73.9125 89.5338) (end 73.9125 88.3457) (width 0.25) (layer "F.Cu") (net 11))
 (segment (start 82.514 90.7948) (end 82.3027 91.0061) (width 0.25) (layer "F.Cu") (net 11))
 (segment (start 75.9141 91.0061) (end 75.1823 90.2743) (width 0.25) (layer "F.Cu") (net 11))
 (segment (start 74.653 90.2743) (end 73.9125 89.5338) (width 0.25) (layer "F.Cu") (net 11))
 (via (at 82.514 90.7948) (size 0.8) (drill 0.4) (layers "F.Cu" "B.Cu") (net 11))
 (segment (start 87.8088 85.5) (end 82.514 90.7948) (width 0.25) (layer "B.Cu") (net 11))
 (segment (start 96 85.5) (end 87.8088 85.5) (width 0.25) (layer "B.Cu") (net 11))
 (segment (start 84.5291 89.5291) (end 85 90) (width 0.25) (layer "F.Cu") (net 1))
 (segment (start 75.8175 89.4726) (end 76.2694 89.9245) (width 0.25) (layer "F.Cu") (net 1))
 (segment (start 86.3158 89.376) (end 85.624 89.376) (width 0.25) (layer "F.Cu") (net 1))
 (segment (start 78.5306 89.9245) (end 78.926 89.5291) (width 0.25) (layer "F.Cu") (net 1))
 (segment (start 78.926 89.5291) (end 84.5291 89.5291) (width 0.25) (layer "F.Cu") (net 1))
 (segment (start 85.624 89.376) (end 85 90) (width 0.25) (layer "F.Cu") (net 1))
 (segment (start 75.8175 88.3457) (end 75.8175 89.4726) (width 0.25) (layer "F.Cu") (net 1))
 (segment (start 76.2694 89.9245) (end 78.5306 89.9245) (width 0.25) (layer "F.Cu") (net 1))
 (via (at 86.3158 89.376) (size 0.8) (drill 0.4) (layers "F.Cu" "B.Cu") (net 1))
 (segment (start 95.955 95.75) (end 92.6898 95.75) (width 0.25) (layer "B.Cu") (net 1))
 (segment (start 92.6898 95.75) (end 86.3158 89.376) (width 0.25) (layer "B.Cu") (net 1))
 (segment (start 74.7711 91.0012) (end 73.2775 92.4948) (width 0.25) (layer "F.Cu") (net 4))
 (segment (start 73.2775 92.4948) (end 73.2775 93.6543) (width 0.25) (layer "F.Cu") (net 4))
 (segment (start 107.91 65.45) (end 103.96 69.4) (width 0.25) (layer "F.Cu") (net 4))
 (segment (start 74.8812 91.0012) (end 74.7711 91.0012) (width 0.25) (layer "F.Cu") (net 4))
 (segment (start 103.96 69.4) (end 89.15 69.4) (width 0.25) (layer "F.Cu") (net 4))
 (via (at 74.8812 91.0012) (size 0.8) (drill 0.4) (layers "F.Cu" "B.Cu") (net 4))
 (segment (start 107.91 65.45) (end 99.5889 65.45) (width 0.25) (layer "B.Cu") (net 4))
 (segment (start 99.5889 65.45) (end 81.9809 83.058) (width 0.25) (layer "B.Cu") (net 4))
 (segment (start 81.9809 83.9015) (end 74.8812 91.0012) (width 0.25) (layer "B.Cu") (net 4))
 (segment (start 81.9809 83.058) (end 81.9809 83.9015) (width 0.25) (layer "B.Cu") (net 4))
 (segment (start 108.5716 97.4705) (end 109.5369 96.5052) (width 0.25) (layer "F.Cu") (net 7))
 (segment (start 78.5068 97.4705) (end 108.5716 97.4705) (width 0.25) (layer "F.Cu") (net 7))
 (segment (start 75.8175 93.6543) (end 75.8175 94.7812) (width 0.25) (layer "F.Cu") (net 7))
 (segment (start 89.3769 76.8769) (end 106.5331 76.8769) (width 0.25) (layer "F.Cu") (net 7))
 (segment (start 75.8175 94.7812) (end 78.5068 97.4705) (width 0.25) (layer "F.Cu") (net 7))
 (segment (start 109.5369 96.5052) (end 109.5369 79.8807) (width 0.25) (layer "F.Cu") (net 7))
 (segment (start 106.5331 76.8769) (end 107.91 75.5) (width 0.25) (layer "F.Cu") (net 7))
 (segment (start 109.5369 79.8807) (end 106.5331 76.8769) (width 0.25) (layer "F.Cu") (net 7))
 (segment (start 88.9 76.4) (end 89.3769 76.8769) (width 0.25) (layer "F.Cu") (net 7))
 (segment (start 89.2845 89) (end 91.7923 86.4922) (width 0.25) (layer "F.Cu") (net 5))
 (segment (start 73.9125 92.5274) (end 74.3683 92.0716) (width 0.25) (layer "F.Cu") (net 5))
 (segment (start 91.7923 86.4922) (end 92.4269 87.1269) (width 0.25) (layer "F.Cu") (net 5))
 (segment (start 73.9125 93.6543) (end 73.9125 92.5274) (width 0.25) (layer "F.Cu") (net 5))
 (segment (start 92.4269 87.1269) (end 106.2331 87.1269) (width 0.25) (layer "F.Cu") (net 5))
 (segment (start 75.3866 91.5238) (end 83.0333 91.5238) (width 0.25) (layer "F.Cu") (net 5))
 (segment (start 86.5497 90.1029) (end 86.6169 90.1029) (width 0.25) (layer "F.Cu") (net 5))
 (segment (start 75.1823 91.7281) (end 75.3866 91.5238) (width 0.25) (layer "F.Cu") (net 5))
 (segment (start 87.7198 89) (end 89.2845 89) (width 0.25) (layer "F.Cu") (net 5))
 (segment (start 88.9 83.6) (end 91.7923 86.4922) (width 0.25) (layer "F.Cu") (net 5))
 (segment (start 86.6169 90.1029) (end 87.7198 89) (width 0.25) (layer "F.Cu") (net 5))
 (segment (start 106.2331 87.1269) (end 107.91 85.45) (width 0.25) (layer "F.Cu") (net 5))
 (segment (start 83.0333 91.5238) (end 83.4852 91.0719) (width 0.25) (layer "F.Cu") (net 5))
 (segment (start 85.5807 91.0719) (end 86.5497 90.1029) (width 0.25) (layer "F.Cu") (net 5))
 (segment (start 83.4852 91.0719) (end 85.5807 91.0719) (width 0.25) (layer "F.Cu") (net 5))
 (segment (start 74.3705 92.0716) (end 74.714 91.7281) (width 0.25) (layer "F.Cu") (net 5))
 (segment (start 74.714 91.7281) (end 75.1823 91.7281) (width 0.25) (layer "F.Cu") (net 5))
 (segment (start 74.3683 92.0716) (end 74.3705 92.0716) (width 0.25) (layer "F.Cu") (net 5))
 (segment (start 75.1825 93.6543) (end 75.1825 92.5274) (width 0.25) (layer "F.Cu") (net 3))
 (segment (start 102.16 90) (end 88.6 90) (width 0.25) (layer "F.Cu") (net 3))
 (segment (start 86.6243 91.9757) (end 88.6 90) (width 0.25) (layer "F.Cu") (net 3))
 (segment (start 75.7342 91.9757) (end 86.6243 91.9757) (width 0.25) (layer "F.Cu") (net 3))
 (segment (start 107.91 95.75) (end 102.16 90) (width 0.25) (layer "F.Cu") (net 3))
 (segment (start 75.1825 92.5274) (end 75.7342 91.9757) (width 0.25) (layer "F.Cu") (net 3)))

